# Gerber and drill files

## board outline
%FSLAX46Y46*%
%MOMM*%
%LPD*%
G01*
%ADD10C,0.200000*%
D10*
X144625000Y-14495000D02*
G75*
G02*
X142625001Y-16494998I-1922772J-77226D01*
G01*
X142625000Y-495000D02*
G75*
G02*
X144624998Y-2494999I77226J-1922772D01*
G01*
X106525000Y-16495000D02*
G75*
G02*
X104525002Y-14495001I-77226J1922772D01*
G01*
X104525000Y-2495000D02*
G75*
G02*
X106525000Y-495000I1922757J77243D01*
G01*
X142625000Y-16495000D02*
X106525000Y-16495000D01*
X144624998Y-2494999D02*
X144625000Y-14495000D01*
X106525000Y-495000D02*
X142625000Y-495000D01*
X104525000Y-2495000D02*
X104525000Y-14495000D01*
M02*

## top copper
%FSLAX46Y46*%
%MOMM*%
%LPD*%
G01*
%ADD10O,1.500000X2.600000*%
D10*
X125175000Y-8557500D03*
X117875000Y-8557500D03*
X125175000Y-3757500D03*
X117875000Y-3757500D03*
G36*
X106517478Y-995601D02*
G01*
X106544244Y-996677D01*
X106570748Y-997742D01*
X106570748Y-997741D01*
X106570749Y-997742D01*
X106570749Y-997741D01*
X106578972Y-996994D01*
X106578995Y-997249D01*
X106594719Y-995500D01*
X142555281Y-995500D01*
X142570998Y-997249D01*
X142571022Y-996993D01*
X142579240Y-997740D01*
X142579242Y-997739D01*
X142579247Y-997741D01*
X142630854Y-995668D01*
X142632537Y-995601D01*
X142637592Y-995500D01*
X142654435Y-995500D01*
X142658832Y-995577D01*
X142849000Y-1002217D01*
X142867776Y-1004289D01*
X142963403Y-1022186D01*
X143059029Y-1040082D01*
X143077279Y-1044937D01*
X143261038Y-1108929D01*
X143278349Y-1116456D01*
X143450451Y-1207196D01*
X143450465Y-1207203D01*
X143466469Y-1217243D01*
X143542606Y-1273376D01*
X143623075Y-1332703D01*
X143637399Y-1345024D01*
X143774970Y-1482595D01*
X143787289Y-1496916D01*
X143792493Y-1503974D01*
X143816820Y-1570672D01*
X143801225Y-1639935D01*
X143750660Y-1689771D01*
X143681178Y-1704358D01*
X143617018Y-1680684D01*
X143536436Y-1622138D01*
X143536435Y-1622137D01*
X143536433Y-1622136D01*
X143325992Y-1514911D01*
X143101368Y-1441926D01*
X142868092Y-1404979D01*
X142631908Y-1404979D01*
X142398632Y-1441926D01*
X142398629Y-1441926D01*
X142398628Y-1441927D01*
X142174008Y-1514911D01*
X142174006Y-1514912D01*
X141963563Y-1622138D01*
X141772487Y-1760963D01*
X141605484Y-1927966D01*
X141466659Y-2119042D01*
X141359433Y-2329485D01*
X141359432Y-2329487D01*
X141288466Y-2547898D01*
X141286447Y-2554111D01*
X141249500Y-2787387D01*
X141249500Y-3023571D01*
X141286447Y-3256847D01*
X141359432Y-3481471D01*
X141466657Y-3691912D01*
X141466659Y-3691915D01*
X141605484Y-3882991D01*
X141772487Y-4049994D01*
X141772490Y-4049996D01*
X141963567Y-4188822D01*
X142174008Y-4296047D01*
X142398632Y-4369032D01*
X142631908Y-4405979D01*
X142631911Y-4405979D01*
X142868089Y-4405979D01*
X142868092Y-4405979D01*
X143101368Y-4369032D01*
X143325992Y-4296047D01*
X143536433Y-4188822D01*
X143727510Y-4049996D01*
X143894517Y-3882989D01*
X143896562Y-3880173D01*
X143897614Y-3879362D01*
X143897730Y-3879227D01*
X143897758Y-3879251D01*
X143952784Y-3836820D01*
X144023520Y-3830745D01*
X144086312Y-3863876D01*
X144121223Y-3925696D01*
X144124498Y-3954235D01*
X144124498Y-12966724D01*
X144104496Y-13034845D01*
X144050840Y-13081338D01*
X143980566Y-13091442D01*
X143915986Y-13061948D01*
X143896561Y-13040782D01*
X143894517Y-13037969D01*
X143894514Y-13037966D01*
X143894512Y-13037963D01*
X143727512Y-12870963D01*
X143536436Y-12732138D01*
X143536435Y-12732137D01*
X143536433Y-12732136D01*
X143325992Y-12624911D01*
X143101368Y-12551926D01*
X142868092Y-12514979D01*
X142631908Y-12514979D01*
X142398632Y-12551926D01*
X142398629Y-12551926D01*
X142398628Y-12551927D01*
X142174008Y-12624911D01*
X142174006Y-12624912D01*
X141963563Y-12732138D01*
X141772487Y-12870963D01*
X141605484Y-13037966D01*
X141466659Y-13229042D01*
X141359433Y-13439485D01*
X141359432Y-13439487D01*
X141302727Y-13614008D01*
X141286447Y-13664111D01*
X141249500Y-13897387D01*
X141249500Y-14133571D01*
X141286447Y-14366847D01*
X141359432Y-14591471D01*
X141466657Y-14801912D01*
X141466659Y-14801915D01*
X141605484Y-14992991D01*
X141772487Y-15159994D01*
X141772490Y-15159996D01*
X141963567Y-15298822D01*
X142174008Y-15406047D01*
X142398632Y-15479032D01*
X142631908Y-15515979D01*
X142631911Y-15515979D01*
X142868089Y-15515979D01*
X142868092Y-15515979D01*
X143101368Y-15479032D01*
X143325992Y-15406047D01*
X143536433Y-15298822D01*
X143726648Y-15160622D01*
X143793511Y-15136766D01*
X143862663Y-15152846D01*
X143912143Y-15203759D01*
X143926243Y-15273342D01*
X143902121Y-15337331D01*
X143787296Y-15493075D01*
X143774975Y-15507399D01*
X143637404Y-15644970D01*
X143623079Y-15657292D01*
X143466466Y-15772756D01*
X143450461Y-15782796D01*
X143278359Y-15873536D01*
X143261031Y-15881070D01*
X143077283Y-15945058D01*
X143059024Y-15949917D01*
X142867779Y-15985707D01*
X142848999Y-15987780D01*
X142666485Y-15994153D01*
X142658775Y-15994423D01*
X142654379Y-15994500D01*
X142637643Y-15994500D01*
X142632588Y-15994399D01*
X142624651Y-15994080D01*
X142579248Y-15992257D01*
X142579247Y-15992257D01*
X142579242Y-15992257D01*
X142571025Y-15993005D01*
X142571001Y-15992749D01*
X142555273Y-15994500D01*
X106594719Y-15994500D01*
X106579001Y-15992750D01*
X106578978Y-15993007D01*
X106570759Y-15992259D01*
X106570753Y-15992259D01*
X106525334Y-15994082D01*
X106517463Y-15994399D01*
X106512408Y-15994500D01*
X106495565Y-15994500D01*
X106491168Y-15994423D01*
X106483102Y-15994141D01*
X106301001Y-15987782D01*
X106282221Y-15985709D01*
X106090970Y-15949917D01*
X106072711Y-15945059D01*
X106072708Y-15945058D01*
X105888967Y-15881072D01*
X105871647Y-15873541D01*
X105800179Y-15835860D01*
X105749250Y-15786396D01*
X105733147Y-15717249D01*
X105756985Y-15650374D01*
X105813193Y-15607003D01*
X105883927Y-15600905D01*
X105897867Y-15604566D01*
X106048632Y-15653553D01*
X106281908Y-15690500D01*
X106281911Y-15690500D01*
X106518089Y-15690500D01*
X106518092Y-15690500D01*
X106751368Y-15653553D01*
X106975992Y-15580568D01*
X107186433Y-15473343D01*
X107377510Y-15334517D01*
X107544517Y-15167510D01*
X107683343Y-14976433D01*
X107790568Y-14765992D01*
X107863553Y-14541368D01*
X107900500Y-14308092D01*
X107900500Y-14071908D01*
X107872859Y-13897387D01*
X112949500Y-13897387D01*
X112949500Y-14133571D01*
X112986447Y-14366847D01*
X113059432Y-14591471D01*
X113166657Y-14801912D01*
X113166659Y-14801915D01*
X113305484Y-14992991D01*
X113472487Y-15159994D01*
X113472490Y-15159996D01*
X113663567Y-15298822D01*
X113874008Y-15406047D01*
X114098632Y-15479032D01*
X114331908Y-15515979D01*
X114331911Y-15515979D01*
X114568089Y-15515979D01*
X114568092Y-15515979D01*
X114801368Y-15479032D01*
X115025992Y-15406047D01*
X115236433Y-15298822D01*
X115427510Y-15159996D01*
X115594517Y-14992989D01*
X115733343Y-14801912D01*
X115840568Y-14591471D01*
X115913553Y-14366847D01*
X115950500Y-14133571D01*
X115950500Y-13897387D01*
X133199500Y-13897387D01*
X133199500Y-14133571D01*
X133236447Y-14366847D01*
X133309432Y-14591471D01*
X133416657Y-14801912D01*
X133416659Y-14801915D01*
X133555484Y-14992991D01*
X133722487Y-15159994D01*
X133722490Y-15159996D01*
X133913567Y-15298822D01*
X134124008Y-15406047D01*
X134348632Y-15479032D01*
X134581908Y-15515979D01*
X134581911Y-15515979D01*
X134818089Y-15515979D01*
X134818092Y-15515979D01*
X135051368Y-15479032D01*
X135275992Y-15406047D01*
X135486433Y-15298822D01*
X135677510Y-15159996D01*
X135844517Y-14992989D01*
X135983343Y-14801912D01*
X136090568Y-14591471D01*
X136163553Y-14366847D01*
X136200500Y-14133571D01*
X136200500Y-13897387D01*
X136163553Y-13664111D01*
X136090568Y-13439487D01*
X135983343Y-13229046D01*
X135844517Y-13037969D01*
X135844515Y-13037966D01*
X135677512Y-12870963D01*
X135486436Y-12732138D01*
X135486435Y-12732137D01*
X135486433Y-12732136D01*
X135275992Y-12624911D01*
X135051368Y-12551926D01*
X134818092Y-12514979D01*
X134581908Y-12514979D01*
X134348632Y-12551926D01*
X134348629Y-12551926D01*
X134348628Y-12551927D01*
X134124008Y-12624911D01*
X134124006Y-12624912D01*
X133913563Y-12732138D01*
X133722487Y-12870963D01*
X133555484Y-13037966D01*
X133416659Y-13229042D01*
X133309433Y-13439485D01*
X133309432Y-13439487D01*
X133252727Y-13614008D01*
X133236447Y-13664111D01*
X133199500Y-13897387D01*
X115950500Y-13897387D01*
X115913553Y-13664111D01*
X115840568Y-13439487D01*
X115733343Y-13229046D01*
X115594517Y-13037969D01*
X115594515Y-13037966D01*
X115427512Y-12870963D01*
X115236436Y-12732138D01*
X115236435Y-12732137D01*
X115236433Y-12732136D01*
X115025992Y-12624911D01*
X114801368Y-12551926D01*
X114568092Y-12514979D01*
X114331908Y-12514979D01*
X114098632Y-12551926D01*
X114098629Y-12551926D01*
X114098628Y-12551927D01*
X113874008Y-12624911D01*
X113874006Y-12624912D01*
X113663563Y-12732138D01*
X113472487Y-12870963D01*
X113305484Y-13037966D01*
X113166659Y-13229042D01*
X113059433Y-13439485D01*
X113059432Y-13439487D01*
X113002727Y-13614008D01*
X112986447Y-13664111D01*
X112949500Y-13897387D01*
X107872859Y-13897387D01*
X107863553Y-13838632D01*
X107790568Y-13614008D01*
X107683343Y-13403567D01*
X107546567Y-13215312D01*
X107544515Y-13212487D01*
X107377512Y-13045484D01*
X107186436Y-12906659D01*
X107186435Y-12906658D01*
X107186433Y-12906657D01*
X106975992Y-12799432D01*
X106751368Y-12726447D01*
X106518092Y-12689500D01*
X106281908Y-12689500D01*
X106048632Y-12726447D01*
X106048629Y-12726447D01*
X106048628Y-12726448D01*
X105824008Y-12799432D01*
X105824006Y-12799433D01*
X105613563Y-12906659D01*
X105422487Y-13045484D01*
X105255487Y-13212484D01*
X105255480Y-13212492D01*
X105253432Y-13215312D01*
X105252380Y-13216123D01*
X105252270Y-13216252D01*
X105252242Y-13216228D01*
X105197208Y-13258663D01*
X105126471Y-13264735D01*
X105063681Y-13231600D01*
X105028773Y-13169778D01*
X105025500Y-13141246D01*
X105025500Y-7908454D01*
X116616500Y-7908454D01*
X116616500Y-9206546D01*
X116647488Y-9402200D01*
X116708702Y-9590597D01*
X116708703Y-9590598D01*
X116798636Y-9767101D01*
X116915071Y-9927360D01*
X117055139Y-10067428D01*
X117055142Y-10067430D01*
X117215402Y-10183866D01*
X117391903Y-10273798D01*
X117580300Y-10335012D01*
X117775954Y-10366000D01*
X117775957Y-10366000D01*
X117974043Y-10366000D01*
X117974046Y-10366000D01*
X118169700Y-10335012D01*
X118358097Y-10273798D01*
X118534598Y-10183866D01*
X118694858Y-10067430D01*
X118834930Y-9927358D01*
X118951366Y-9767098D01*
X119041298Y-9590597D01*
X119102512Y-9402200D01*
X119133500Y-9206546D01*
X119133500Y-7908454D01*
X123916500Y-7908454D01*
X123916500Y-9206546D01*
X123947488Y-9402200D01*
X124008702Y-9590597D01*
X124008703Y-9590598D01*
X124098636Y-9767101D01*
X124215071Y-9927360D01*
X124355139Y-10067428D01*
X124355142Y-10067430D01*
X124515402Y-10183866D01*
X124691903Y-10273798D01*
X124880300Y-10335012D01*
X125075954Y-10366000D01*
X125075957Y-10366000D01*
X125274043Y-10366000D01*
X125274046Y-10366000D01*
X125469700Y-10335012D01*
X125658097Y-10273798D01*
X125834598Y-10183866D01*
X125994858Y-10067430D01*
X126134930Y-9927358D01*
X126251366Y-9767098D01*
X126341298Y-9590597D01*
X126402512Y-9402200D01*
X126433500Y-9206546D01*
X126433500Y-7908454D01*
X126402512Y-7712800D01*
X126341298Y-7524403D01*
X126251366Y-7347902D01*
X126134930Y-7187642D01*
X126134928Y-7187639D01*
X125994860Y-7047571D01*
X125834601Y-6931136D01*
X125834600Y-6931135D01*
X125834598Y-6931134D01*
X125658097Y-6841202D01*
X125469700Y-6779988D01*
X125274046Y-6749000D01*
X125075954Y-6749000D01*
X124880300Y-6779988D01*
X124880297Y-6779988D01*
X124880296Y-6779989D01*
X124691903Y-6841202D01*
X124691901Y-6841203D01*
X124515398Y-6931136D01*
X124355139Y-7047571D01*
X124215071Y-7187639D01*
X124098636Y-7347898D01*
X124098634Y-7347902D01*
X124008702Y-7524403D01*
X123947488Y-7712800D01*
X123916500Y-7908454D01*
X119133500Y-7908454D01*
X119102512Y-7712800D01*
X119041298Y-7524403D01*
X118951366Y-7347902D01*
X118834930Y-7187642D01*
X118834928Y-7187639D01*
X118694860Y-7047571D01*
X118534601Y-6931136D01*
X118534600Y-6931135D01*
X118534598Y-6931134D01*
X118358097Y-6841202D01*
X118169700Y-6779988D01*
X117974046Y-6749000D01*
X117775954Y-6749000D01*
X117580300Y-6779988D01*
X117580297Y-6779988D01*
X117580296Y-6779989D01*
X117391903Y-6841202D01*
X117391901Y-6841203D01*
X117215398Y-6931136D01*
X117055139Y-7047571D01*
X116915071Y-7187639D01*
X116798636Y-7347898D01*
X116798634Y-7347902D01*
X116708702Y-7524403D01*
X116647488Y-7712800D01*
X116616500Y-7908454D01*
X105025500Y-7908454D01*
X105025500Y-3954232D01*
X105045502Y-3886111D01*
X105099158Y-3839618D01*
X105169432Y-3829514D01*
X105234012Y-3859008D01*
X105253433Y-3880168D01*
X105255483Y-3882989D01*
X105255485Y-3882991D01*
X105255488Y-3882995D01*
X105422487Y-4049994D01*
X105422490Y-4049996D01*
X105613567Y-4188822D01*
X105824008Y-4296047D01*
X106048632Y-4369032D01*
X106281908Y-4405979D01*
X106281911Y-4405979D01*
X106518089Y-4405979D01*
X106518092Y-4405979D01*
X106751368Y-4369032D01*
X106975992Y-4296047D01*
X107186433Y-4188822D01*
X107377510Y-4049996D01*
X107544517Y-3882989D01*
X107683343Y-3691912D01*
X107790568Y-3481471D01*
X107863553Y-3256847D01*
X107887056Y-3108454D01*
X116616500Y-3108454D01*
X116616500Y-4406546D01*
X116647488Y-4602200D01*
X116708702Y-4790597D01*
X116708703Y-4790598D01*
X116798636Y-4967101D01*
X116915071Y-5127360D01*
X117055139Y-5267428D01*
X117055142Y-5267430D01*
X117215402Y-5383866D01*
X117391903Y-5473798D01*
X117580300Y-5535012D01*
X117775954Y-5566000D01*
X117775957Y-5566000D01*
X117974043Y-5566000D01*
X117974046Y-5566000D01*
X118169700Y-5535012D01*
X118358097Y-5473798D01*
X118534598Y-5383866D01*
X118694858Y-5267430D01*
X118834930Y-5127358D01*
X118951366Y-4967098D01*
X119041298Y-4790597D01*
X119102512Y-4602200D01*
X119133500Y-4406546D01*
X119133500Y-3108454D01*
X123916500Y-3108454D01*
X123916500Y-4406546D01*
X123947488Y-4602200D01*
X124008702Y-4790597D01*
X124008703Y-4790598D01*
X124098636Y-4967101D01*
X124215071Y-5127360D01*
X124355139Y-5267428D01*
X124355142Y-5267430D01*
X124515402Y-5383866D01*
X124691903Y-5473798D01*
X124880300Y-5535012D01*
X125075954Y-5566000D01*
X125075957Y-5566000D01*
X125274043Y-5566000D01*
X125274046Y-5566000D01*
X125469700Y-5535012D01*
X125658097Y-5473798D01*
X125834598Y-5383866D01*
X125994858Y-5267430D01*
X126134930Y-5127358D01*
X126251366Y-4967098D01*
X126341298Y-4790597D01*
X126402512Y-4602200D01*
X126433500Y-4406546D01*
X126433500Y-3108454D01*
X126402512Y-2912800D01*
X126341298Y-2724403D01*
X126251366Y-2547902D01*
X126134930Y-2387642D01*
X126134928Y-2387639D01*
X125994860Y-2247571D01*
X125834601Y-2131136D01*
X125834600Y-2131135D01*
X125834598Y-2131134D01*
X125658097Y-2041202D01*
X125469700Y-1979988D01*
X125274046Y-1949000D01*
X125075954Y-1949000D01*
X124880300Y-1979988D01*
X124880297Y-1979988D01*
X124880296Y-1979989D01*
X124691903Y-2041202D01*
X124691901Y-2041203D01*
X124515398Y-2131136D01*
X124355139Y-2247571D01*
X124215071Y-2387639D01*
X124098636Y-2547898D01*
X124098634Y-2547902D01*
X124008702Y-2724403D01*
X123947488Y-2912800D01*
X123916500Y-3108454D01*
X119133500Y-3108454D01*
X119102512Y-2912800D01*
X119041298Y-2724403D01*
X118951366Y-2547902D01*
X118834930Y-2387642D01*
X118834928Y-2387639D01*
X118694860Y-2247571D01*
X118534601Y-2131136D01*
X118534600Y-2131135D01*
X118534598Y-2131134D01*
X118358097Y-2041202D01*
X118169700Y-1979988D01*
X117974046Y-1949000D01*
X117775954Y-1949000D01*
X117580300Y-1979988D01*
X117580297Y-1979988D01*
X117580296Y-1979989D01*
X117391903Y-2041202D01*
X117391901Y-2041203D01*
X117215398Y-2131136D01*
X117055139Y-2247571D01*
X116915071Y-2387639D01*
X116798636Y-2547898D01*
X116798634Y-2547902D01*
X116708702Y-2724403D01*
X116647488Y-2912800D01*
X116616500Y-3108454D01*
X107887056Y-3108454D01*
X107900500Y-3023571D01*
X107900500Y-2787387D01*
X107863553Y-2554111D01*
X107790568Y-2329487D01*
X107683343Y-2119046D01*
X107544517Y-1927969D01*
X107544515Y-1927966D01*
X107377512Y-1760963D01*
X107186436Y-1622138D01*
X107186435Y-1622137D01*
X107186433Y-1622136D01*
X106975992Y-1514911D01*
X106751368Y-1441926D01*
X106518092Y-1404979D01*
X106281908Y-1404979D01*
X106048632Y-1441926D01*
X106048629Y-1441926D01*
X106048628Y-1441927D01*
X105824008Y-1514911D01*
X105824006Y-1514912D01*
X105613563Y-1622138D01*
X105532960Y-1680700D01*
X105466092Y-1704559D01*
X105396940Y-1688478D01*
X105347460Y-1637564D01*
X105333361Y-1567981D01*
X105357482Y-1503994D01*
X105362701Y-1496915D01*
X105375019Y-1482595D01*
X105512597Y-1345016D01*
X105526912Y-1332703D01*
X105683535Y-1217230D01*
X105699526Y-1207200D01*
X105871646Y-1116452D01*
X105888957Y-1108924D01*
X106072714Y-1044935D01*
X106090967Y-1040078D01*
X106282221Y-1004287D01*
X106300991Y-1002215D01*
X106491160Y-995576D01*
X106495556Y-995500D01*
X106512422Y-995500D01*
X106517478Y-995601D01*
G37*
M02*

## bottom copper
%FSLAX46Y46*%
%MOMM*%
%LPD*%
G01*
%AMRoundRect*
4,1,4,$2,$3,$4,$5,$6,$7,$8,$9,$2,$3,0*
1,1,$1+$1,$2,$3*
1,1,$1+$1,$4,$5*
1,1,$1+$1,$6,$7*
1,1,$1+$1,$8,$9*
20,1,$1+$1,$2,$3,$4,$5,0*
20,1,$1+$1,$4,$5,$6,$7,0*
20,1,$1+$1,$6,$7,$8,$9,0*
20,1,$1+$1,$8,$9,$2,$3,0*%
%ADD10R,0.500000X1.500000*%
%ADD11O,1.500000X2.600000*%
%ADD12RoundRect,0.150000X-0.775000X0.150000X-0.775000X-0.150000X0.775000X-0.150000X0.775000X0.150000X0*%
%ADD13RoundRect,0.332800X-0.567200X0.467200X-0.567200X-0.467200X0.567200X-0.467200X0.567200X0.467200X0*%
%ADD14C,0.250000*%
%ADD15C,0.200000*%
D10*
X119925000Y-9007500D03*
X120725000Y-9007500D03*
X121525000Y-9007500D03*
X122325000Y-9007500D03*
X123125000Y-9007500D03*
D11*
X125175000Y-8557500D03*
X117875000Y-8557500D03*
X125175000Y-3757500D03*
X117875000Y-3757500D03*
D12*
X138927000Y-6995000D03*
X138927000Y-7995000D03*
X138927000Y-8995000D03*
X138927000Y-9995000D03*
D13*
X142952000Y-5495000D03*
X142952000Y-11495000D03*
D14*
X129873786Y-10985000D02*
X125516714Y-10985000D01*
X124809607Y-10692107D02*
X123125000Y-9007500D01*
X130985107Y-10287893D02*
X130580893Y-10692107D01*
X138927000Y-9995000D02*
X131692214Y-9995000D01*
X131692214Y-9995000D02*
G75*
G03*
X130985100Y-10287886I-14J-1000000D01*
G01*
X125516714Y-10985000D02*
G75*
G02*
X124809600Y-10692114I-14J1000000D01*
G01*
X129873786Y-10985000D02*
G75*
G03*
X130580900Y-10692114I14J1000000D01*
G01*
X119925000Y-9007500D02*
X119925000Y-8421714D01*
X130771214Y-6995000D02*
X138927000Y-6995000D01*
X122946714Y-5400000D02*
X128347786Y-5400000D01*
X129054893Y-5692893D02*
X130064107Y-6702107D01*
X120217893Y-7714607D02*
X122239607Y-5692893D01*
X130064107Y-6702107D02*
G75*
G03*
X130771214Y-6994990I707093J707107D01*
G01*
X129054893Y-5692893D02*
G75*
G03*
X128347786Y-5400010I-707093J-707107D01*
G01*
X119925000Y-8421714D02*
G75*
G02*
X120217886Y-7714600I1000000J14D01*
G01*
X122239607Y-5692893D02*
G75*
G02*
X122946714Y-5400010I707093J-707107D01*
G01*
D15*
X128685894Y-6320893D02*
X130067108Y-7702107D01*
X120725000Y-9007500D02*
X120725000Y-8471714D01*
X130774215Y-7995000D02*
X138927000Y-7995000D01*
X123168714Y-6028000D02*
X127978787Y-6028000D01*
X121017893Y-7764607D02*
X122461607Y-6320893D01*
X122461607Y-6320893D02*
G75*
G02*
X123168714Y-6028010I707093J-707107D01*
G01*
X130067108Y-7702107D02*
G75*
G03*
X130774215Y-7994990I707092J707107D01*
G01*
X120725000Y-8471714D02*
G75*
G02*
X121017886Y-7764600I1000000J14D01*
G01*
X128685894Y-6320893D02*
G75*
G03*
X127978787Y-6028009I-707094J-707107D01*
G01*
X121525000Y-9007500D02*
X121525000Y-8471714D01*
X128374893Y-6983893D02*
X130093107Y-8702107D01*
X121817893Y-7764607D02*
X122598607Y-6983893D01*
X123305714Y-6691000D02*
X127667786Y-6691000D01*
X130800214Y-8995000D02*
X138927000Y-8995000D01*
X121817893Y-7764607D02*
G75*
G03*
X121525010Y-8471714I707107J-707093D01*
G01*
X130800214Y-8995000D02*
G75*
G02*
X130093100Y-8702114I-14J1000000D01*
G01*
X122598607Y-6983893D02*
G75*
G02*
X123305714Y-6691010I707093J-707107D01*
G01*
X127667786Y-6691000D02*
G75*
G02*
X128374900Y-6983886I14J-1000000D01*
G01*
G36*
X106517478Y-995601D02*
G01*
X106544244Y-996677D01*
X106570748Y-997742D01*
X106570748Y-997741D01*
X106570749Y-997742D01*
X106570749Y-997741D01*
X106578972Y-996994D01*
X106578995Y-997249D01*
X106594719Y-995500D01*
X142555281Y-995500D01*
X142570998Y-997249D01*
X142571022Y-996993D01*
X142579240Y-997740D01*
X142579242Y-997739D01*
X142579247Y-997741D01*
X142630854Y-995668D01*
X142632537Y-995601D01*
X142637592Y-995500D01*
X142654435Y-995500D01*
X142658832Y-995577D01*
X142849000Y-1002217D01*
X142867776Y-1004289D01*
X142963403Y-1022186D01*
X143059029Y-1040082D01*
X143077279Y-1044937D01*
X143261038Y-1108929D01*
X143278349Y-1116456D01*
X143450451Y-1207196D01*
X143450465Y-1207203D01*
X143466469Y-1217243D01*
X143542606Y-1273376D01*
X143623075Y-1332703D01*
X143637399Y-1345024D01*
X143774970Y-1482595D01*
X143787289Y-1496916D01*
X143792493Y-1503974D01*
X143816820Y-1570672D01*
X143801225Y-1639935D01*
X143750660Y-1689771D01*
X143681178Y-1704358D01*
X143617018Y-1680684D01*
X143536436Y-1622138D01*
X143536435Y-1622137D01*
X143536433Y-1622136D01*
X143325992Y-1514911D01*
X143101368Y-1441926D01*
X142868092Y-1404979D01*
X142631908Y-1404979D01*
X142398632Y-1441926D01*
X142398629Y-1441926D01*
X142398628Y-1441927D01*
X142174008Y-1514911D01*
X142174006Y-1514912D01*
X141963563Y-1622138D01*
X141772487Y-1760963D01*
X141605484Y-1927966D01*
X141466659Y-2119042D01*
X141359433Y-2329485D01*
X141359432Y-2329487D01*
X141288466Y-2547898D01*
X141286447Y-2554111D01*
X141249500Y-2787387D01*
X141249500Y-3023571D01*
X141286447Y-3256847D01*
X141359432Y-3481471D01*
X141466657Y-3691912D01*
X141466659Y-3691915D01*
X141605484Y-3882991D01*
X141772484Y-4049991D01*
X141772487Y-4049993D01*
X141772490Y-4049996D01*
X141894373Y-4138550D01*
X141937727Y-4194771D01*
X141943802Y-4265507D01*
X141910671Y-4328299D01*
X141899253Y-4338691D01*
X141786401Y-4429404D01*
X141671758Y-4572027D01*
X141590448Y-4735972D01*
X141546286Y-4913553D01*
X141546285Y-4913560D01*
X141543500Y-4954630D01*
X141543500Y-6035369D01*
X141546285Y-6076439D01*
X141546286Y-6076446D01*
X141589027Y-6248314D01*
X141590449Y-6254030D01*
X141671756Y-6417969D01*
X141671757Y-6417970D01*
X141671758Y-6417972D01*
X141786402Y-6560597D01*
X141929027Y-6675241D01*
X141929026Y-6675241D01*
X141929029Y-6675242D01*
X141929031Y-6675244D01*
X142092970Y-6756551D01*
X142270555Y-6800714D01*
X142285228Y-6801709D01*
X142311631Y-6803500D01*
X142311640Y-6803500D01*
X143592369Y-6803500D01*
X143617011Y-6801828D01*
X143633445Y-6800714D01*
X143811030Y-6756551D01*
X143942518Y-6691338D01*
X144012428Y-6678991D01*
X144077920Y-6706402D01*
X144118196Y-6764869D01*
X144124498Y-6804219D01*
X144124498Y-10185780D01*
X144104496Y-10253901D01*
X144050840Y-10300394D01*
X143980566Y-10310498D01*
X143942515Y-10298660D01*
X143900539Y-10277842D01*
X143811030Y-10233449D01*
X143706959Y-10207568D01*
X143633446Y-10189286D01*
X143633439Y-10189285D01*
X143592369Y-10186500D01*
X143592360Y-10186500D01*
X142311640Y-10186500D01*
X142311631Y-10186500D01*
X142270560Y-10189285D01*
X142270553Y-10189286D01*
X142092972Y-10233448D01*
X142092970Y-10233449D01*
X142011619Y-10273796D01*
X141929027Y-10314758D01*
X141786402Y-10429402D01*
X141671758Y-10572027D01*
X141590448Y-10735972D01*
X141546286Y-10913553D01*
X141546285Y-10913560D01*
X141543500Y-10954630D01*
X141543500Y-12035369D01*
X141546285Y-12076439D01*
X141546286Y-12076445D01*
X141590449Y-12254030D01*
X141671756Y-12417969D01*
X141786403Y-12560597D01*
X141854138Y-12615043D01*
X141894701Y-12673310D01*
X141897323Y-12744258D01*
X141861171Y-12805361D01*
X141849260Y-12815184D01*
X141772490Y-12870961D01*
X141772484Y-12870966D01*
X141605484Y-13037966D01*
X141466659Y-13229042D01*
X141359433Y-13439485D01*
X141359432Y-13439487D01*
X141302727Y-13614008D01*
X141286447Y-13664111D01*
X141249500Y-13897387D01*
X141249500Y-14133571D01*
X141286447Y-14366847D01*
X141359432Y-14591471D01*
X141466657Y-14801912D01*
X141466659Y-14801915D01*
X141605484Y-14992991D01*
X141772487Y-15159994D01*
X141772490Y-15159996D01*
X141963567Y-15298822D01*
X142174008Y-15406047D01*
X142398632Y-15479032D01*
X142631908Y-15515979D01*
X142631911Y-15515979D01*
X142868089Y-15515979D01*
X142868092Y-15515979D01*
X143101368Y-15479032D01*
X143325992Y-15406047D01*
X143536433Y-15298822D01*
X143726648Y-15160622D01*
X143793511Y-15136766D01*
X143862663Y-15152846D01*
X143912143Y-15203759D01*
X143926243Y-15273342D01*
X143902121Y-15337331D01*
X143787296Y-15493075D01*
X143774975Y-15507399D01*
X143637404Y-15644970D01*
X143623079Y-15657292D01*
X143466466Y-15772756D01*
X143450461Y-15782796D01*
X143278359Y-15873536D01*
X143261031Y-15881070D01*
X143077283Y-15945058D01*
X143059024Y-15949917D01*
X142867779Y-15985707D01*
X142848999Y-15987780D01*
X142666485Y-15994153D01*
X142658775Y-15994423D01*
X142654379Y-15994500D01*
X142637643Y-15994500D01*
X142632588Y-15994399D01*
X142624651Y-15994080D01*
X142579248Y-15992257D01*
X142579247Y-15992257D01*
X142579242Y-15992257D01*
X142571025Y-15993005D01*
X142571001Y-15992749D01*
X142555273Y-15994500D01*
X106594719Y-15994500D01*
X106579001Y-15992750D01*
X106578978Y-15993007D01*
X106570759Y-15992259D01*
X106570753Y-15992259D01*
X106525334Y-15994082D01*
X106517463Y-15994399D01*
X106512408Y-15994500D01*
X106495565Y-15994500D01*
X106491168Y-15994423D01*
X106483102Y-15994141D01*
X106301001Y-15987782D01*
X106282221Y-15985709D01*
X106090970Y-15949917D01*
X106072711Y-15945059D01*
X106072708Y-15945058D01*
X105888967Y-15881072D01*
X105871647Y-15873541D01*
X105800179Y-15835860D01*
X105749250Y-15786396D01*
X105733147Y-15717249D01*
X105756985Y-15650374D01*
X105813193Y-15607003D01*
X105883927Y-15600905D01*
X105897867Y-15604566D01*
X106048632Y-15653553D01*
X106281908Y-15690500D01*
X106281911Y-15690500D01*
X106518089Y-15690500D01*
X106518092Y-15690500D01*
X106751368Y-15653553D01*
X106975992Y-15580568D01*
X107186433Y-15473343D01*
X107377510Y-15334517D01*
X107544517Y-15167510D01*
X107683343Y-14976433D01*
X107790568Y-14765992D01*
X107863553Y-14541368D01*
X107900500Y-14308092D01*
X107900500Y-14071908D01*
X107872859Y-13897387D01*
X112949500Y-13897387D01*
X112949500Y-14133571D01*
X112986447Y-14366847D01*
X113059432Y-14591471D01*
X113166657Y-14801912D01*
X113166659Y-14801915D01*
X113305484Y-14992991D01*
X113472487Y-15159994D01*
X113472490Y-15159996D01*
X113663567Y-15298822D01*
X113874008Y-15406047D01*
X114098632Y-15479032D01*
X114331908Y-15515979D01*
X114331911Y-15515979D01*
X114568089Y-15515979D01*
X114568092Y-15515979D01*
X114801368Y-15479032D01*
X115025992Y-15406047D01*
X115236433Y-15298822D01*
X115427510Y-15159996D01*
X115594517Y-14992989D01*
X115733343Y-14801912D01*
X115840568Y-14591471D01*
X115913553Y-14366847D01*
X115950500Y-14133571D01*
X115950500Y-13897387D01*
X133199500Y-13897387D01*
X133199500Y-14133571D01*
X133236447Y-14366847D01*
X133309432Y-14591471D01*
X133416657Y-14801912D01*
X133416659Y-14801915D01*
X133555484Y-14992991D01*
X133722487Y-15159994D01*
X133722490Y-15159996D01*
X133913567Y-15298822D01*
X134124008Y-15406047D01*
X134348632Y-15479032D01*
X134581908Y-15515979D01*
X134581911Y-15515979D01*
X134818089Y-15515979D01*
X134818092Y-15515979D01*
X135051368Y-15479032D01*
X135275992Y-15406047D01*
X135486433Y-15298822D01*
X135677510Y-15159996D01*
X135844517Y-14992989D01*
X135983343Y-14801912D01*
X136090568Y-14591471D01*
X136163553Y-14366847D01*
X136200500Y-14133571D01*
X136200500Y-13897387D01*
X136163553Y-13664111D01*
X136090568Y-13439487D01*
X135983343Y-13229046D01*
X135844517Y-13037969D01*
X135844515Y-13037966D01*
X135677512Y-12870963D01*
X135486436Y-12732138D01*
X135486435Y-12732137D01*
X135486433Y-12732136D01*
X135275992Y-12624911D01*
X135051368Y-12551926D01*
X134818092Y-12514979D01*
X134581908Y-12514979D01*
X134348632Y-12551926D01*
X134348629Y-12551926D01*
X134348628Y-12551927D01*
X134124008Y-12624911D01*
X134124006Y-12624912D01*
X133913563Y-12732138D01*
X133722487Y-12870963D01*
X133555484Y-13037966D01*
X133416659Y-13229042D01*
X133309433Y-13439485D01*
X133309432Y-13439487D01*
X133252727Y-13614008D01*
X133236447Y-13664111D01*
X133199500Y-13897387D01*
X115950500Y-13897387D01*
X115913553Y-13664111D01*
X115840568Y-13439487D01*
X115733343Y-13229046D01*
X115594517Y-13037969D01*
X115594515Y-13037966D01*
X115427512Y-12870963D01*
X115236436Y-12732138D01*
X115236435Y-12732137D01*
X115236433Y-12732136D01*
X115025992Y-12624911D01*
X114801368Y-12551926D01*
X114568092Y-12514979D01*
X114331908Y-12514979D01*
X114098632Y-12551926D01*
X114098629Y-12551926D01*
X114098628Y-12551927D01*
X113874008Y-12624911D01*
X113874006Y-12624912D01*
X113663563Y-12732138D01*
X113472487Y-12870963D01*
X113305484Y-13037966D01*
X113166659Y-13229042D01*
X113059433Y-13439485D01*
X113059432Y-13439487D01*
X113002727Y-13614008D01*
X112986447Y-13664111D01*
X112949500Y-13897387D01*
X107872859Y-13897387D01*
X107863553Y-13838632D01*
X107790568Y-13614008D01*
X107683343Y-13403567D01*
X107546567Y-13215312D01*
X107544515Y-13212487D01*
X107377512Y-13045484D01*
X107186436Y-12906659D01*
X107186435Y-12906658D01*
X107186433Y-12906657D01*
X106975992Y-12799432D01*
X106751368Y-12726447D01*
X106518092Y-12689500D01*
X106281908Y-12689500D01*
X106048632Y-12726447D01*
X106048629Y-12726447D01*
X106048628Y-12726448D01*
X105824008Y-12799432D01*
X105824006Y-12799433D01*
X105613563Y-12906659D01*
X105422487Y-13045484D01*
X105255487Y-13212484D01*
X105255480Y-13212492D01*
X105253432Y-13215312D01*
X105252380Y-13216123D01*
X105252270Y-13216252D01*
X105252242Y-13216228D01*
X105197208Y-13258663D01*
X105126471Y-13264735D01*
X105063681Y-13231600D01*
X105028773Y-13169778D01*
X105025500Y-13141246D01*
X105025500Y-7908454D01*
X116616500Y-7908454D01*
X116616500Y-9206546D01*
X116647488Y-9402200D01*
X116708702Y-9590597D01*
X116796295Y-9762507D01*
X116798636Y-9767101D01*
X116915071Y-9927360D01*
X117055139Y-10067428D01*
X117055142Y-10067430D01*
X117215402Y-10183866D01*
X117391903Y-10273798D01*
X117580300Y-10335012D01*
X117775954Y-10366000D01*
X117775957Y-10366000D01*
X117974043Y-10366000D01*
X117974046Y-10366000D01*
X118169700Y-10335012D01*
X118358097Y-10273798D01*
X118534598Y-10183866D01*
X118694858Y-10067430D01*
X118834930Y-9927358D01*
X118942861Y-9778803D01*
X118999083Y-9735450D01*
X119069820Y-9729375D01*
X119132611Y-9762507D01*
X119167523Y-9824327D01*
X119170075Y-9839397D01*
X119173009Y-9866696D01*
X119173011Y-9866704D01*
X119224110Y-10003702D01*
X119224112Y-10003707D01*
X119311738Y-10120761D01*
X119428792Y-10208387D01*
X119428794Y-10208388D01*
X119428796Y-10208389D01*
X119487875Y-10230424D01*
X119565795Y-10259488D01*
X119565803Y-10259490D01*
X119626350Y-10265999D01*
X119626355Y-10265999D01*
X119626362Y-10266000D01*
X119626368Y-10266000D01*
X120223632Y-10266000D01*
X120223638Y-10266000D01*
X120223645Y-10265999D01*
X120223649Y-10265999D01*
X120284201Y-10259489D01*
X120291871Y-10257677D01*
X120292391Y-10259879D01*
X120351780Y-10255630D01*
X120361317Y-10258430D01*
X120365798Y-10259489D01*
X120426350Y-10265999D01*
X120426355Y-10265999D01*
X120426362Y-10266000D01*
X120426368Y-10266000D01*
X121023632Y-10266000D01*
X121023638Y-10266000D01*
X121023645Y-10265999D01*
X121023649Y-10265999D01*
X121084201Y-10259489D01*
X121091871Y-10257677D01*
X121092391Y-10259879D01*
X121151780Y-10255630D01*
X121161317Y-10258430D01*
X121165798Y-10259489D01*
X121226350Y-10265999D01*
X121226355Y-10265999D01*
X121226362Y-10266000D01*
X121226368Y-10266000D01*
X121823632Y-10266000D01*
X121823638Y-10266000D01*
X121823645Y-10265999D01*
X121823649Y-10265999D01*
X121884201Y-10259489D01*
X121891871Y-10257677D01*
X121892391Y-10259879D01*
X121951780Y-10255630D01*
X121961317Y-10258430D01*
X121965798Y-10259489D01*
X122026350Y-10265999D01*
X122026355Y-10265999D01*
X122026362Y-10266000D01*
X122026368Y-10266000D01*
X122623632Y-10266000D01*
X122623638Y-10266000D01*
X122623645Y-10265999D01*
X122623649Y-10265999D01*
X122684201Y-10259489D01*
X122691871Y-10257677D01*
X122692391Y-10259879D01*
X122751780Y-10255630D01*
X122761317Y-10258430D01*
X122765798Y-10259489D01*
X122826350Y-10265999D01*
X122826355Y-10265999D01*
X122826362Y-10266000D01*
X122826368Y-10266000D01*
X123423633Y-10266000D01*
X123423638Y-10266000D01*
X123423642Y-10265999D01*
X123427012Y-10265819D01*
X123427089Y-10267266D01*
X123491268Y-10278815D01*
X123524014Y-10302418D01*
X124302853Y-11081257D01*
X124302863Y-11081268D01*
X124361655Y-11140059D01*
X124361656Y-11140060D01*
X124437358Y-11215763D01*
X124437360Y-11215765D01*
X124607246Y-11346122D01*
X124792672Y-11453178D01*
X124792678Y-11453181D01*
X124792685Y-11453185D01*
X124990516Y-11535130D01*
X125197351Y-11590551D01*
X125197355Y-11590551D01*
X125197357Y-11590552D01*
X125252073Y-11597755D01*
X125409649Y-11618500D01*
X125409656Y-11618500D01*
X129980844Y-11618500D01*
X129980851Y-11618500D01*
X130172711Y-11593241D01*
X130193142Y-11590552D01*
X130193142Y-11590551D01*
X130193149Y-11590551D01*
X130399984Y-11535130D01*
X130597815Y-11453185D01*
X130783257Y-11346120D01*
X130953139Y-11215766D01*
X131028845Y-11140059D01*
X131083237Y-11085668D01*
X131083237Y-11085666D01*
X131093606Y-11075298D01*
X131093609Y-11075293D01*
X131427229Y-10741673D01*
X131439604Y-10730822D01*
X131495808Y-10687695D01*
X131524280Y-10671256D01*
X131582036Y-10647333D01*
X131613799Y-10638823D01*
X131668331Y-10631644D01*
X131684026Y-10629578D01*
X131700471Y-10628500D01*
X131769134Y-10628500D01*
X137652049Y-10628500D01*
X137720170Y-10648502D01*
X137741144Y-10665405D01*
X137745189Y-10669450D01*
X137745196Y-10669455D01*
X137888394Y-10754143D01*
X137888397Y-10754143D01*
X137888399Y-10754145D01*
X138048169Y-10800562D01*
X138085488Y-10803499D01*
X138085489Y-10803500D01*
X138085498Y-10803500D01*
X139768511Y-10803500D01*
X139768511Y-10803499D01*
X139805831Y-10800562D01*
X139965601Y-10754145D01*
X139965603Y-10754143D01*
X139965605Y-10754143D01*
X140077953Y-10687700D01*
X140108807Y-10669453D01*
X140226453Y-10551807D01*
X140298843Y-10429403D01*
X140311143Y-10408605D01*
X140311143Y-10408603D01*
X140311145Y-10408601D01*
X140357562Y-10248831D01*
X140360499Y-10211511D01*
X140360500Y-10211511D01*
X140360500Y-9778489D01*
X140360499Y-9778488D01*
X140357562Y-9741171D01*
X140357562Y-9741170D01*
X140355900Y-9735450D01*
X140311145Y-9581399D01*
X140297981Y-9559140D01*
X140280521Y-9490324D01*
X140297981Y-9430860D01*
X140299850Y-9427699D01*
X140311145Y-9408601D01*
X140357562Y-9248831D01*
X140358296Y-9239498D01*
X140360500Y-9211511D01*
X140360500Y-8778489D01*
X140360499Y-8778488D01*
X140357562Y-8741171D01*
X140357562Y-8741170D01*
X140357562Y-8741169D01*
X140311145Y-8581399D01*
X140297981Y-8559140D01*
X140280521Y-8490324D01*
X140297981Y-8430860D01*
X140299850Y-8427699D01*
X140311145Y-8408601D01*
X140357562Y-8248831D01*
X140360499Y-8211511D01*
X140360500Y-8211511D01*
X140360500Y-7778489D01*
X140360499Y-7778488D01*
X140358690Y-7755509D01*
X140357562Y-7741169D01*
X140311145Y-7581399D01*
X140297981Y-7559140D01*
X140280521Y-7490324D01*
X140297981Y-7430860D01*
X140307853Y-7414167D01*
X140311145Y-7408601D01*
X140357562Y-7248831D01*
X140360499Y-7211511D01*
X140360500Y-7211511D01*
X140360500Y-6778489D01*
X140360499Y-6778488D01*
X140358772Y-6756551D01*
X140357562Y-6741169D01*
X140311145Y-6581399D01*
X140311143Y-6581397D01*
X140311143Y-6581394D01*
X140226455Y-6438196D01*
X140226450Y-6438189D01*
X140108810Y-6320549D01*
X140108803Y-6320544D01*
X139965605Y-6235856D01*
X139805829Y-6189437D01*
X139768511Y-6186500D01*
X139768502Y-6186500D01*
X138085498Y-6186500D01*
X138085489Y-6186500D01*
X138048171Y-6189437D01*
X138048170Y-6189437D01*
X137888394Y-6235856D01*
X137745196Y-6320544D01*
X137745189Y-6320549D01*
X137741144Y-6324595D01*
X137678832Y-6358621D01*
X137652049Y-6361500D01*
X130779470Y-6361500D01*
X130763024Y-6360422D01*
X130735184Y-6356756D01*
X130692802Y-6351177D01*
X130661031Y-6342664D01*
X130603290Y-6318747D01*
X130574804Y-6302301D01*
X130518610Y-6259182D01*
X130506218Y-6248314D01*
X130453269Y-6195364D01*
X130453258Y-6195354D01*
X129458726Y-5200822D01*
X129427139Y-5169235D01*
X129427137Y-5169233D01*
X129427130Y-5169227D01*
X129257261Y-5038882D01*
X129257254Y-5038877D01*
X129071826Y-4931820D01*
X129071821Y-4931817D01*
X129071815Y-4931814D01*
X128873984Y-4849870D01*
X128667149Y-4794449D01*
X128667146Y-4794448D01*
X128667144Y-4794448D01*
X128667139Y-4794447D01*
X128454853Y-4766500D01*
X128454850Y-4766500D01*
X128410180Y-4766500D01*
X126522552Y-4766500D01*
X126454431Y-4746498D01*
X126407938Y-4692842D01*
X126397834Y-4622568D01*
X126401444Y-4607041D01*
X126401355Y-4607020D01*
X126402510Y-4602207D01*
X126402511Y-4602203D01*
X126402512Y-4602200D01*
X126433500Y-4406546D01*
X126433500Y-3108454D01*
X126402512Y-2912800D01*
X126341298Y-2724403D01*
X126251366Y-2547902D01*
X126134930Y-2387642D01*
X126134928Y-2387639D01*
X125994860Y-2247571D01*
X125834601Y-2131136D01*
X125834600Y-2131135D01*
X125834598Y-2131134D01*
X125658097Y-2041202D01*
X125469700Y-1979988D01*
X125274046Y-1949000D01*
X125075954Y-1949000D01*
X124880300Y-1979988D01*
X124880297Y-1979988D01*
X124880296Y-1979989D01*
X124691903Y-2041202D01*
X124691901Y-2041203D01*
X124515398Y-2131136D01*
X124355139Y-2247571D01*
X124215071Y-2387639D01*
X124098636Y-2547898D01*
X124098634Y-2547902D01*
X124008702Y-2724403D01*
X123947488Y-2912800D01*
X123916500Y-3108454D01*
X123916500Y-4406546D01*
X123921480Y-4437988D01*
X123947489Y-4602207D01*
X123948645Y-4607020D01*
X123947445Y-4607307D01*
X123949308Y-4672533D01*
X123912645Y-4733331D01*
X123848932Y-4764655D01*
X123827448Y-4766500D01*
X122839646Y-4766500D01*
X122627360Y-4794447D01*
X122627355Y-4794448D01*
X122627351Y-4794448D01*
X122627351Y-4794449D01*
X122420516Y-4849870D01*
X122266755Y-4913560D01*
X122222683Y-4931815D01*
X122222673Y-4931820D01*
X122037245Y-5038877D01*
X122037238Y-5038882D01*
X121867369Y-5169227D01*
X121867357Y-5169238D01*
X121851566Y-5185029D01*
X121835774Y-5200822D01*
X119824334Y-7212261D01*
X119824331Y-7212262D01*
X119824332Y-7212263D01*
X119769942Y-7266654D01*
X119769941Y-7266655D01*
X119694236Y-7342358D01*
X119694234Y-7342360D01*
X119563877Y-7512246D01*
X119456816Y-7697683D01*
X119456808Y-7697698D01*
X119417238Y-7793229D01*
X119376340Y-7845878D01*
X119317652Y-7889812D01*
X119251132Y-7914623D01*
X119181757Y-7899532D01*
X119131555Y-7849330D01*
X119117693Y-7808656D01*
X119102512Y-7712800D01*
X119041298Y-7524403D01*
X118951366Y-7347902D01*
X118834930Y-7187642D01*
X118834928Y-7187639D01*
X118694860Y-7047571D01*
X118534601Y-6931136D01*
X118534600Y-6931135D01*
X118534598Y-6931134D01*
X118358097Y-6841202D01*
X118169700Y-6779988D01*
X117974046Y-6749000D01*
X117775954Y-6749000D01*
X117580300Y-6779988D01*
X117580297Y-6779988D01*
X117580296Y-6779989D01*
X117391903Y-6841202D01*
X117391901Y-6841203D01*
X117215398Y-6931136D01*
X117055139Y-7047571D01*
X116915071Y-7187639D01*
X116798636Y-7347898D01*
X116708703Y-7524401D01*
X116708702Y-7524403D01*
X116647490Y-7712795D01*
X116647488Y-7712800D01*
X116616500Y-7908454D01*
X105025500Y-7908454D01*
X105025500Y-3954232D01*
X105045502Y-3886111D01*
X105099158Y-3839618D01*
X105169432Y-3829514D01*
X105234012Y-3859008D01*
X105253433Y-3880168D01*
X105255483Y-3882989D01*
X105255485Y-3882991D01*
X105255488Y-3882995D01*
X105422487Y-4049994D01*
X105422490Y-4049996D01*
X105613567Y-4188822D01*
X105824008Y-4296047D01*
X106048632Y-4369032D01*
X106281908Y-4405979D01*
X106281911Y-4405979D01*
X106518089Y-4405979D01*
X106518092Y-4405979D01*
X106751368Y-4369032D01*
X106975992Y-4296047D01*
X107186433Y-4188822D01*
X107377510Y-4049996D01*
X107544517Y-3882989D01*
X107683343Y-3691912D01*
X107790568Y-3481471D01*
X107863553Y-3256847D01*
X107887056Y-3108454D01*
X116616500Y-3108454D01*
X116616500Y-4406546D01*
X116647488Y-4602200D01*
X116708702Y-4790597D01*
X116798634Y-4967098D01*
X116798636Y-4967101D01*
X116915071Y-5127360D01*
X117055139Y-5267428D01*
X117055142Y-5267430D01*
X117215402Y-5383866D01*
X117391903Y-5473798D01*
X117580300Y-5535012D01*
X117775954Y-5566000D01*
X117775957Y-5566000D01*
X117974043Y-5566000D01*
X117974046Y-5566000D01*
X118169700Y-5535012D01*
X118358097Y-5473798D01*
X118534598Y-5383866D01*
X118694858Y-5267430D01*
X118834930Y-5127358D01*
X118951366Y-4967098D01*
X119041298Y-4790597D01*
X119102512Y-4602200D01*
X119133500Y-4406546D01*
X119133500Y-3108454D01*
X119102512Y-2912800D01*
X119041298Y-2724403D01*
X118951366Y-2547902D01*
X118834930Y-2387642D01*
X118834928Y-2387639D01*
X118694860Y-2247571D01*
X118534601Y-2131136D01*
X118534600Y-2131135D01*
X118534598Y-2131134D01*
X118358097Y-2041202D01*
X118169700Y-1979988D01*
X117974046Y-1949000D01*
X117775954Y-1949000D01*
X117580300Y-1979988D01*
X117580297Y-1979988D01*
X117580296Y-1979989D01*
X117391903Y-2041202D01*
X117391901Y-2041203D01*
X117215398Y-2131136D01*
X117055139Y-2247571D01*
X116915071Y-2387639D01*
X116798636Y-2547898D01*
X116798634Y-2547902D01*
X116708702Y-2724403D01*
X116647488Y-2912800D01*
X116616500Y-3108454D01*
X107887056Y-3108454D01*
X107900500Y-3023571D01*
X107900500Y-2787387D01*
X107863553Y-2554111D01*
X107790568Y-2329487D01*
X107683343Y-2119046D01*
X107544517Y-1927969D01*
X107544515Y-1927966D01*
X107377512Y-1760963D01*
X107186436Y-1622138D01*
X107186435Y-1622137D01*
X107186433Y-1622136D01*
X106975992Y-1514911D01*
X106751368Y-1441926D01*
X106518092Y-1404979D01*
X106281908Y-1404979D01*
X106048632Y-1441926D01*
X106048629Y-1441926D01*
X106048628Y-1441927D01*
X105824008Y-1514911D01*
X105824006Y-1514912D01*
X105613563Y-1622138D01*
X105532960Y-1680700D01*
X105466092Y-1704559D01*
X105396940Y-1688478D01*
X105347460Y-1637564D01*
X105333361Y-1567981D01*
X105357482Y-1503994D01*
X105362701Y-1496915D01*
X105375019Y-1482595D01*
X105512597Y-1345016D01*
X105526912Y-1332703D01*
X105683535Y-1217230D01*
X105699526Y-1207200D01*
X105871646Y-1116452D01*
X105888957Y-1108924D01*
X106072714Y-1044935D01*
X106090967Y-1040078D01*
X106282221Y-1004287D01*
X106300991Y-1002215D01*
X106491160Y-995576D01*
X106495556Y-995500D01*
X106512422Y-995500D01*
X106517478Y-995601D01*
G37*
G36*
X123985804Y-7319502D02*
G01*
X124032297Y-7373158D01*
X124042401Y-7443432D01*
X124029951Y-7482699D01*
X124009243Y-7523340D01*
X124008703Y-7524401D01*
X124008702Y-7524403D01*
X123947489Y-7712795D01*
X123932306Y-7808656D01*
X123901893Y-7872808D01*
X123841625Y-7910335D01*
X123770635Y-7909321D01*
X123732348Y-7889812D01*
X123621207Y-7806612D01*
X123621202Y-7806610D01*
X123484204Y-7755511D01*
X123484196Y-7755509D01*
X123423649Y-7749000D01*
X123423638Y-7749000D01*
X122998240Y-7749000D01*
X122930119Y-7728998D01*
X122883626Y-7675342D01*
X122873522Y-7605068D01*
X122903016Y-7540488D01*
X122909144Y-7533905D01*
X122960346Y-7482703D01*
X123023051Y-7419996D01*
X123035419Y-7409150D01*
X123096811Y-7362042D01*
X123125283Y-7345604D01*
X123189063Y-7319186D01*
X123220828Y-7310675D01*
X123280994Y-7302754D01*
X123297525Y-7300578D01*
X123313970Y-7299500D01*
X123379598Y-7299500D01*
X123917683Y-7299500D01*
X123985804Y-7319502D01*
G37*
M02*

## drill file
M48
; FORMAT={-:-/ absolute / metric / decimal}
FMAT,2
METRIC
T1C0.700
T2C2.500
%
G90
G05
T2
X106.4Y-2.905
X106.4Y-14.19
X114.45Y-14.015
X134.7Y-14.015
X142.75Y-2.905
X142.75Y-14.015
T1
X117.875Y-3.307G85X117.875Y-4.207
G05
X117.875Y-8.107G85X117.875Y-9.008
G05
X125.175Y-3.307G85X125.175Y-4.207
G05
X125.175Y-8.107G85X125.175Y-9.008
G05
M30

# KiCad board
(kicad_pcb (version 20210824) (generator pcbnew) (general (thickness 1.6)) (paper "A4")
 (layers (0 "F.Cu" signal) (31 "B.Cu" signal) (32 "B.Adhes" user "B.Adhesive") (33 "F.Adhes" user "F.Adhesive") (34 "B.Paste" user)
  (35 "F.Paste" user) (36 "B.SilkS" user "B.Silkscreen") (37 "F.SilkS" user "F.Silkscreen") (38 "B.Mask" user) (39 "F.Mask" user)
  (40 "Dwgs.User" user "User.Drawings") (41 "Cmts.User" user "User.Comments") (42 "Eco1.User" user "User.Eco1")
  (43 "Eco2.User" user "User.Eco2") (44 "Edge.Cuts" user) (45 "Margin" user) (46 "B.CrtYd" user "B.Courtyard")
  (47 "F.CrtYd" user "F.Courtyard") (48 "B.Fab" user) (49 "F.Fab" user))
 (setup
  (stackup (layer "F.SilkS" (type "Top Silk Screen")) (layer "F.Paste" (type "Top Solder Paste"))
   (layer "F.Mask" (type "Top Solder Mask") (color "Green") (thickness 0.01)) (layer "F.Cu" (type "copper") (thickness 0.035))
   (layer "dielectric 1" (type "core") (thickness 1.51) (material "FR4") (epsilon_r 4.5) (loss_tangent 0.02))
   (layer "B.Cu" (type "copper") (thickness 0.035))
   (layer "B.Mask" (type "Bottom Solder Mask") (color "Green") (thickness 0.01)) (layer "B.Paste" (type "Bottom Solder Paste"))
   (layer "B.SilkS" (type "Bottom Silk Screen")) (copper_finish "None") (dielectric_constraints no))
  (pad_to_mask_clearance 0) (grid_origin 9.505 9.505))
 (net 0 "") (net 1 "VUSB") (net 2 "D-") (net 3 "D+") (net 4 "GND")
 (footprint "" (layer "F.Cu") (at 136.255 14.205)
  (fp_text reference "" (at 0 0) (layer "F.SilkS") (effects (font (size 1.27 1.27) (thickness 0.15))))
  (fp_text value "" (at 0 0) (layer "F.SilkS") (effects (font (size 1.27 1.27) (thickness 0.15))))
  (pad "" np_thru_hole circle (at -1.555 -0.189521) (size 2.5 2.5) (drill 2.5) (layers F&B.Cu *.Mask)))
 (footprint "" (layer "F.Cu") (at 94.555 1.535)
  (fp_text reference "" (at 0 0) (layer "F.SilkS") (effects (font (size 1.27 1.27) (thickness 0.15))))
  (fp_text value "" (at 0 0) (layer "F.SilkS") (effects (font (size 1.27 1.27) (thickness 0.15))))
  (pad "" np_thru_hole circle (at 11.845 1.370479) (size 2.5 2.5) (drill 2.5) (layers F&B.Cu *.Mask)))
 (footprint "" (layer "F.Cu") (at 147.015 3.065)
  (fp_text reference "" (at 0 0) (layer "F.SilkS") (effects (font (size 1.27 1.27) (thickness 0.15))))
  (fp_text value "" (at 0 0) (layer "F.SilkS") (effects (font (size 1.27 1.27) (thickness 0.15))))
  (pad "" np_thru_hole circle (at -4.265 -0.159521) (size 2.5 2.5) (drill 2.5) (layers F&B.Cu *.Mask)))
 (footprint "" (layer "F.Cu") (at 94.295 7.445633)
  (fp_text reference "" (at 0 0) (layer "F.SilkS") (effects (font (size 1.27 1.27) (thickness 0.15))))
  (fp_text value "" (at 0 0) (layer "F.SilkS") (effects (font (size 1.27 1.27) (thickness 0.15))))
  (pad "" np_thru_hole circle (at 12.105 6.744367) (size 2.5 2.5) (drill 2.5) (layers F&B.Cu *.Mask)))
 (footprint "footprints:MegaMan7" (layer "F.Cu") (at 109.650838 8.415023)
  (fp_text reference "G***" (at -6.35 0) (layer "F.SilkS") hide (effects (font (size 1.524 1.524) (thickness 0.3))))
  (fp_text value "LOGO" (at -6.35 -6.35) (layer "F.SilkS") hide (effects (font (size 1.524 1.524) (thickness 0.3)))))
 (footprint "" (layer "F.Cu") (at 112.225 13.965)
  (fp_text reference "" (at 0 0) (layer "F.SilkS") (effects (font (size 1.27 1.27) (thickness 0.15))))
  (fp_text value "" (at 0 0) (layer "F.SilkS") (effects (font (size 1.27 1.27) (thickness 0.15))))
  (pad "" np_thru_hole circle (at 2.225 0.050479) (size 2.5 2.5) (drill 2.5) (layers F&B.Cu *.Mask)))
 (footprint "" (layer "F.Cu") (at 130.75 14.19)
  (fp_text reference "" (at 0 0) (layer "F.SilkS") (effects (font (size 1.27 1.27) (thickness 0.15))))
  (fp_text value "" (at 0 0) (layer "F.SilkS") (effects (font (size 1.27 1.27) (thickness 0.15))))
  (pad "" np_thru_hole circle (at 12 -0.174521) (size 2.5 2.5) (drill 2.5) (layers F&B.Cu *.Mask)))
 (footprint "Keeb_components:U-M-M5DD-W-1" (layer "B.Cu") (at 121.525 3.7575 180)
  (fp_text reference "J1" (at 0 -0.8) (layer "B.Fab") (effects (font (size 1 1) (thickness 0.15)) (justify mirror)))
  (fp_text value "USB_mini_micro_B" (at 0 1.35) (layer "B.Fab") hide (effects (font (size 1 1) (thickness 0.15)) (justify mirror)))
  (pad "1" smd rect locked (at 1.6 -5.25) (size 0.5 1.5) (layers "B.Cu" "B.Paste" "B.Mask") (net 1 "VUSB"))
  (pad "2" smd rect locked (at 0.8 -5.25) (size 0.5 1.5) (layers "B.Cu" "B.Paste" "B.Mask") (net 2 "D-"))
  (pad "3" smd rect locked (at 0 -5.25) (size 0.5 1.5) (layers "B.Cu" "B.Paste" "B.Mask") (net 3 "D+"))
  (pad "4" smd rect locked (at -0.8 -5.25) (size 0.5 1.5) (layers "B.Cu" "B.Paste" "B.Mask"))
  (pad "5" smd rect locked (at -1.6 -5.25) (size 0.5 1.5) (layers "B.Cu" "B.Paste" "B.Mask") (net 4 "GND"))
  (pad "6" thru_hole oval locked (at -3.65 -4.8) (size 1.5 2.6) (drill oval 0.7 1.6) (layers *.Cu *.Mask))
  (pad "6" thru_hole oval locked (at 3.65 -4.8) (size 1.5 2.6) (drill oval 0.7 1.6) (layers *.Cu *.Mask))
  (pad "6" thru_hole oval locked (at -3.65 0) (size 1.5 2.6) (drill oval 0.7 1.6) (layers *.Cu *.Mask))
  (pad "6" thru_hole oval locked (at 3.65 0) (size 1.5 2.6) (drill oval 0.7 1.6) (layers *.Cu *.Mask)))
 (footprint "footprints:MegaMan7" (layer "B.Cu") (at 109.67284 8.39588 180)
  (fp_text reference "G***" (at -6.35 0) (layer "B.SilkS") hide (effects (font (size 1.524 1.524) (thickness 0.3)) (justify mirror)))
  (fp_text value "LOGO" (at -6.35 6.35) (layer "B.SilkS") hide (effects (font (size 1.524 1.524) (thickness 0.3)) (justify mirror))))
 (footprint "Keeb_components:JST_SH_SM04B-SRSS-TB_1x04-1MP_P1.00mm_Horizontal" (layer "B.Cu") (at 141.077 8.495 -90)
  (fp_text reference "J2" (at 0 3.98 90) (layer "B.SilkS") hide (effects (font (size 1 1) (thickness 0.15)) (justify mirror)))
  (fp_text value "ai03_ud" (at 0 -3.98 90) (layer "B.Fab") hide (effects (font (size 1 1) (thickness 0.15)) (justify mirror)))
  (pad "1" smd roundrect locked (at -1.5 2.15 270) (size 0.6 1.85) (layers "B.Cu" "B.Paste" "B.Mask") (roundrect_rratio 0.25) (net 1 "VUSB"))
  (pad "2" smd roundrect locked (at -0.5 2.15 270) (size 0.6 1.85) (layers "B.Cu" "B.Paste" "B.Mask") (roundrect_rratio 0.25) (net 2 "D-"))
  (pad "3" smd roundrect locked (at 0.5 2.15 270) (size 0.6 1.85) (layers "B.Cu" "B.Paste" "B.Mask") (roundrect_rratio 0.25) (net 3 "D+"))
  (pad "4" smd roundrect locked (at 1.5 2.15 270) (size 0.6 1.85) (layers "B.Cu" "B.Paste" "B.Mask") (roundrect_rratio 0.25) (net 4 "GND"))
  (pad "MP" smd roundrect locked (at -3 -1.875 270) (size 1.6 1.8) (layers "B.Cu" "B.Paste" "B.Mask") (roundrect_rratio 0.208))
  (pad "MP" smd roundrect locked (at 3 -1.875 270) (size 1.6 1.8) (layers "B.Cu" "B.Paste" "B.Mask") (roundrect_rratio 0.208)))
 (gr_arc (start 142.702228 14.572226) (end 144.625 14.495) (angle 94.6) (layer "Edge.Cuts") (width 0.2))
 (gr_arc (start 142.702226 2.417772) (end 142.625 0.495) (angle 94.6) (layer "Edge.Cuts") (width 0.2))
 (gr_arc (start 106.447774 14.572228) (end 106.525 16.495) (angle 94.6) (layer "Edge.Cuts") (width 0.2))
 (gr_arc (start 106.447757 2.417757) (end 104.525 2.495) (angle 94.60101756) (layer "Edge.Cuts") (width 0.2))
 (gr_line (start 142.625 16.495) (end 106.525 16.495) (layer "Edge.Cuts") (width 0.2))
 (gr_line (start 144.624998 2.494999) (end 144.625 14.495) (layer "Edge.Cuts") (width 0.2))
 (gr_line (start 106.525 0.495) (end 142.625 0.495) (layer "Edge.Cuts") (width 0.2))
 (gr_line (start 104.525 2.495) (end 104.525 14.495) (layer "Edge.Cuts") (width 0.2))
 (segment (start 129.873786 10.985) (end 125.516714 10.985) (width 0.25) (layer "B.Cu") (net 4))
 (segment (start 124.809607 10.692107) (end 123.125 9.0075) (width 0.25) (layer "B.Cu") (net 4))
 (segment (start 130.985107 10.287893) (end 130.580893 10.692107) (width 0.25) (layer "B.Cu") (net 4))
 (segment (start 138.927 9.995) (end 131.692214 9.995) (width 0.25) (layer "B.Cu") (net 4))
 (arc (start 131.692214 9.995) (mid 131.309531 10.07112) (end 130.985107 10.287893) (width 0.25) (layer "B.Cu") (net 4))
 (arc (start 125.516714 10.985) (mid 125.134031 10.90888) (end 124.809607 10.692107) (width 0.25) (layer "B.Cu") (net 4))
 (arc (start 129.873786 10.985) (mid 130.256469 10.90888) (end 130.580893 10.692107) (width 0.25) (layer "B.Cu") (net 4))
 (segment (start 119.925 9.0075) (end 119.925 8.421714) (width 0.25) (layer "B.Cu") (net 1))
 (segment (start 130.771214 6.995) (end 138.927 6.995) (width 0.25) (layer "B.Cu") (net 1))
 (segment (start 122.946714 5.4) (end 128.347786 5.4) (width 0.25) (layer "B.Cu") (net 1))
 (segment (start 129.054893 5.692893) (end 130.064107 6.702107) (width 0.25) (layer "B.Cu") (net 1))
 (segment (start 120.217893 7.714607) (end 122.239607 5.692893) (width 0.25) (layer "B.Cu") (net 1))
 (arc (start 130.064107 6.702107) (mid 130.38853 6.91888) (end 130.771214 6.995) (width 0.25) (layer "B.Cu") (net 1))
 (arc (start 129.054893 5.692893) (mid 128.73047 5.47612) (end 128.347786 5.4) (width 0.25) (layer "B.Cu") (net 1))
 (arc (start 119.925 8.421714) (mid 120.00112 8.039031) (end 120.217893 7.714607) (width 0.25) (layer "B.Cu") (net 1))
 (arc (start 122.239607 5.692893) (mid 122.56403 5.47612) (end 122.946714 5.4) (width 0.25) (layer "B.Cu") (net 1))
 (segment (start 128.685894 6.320893) (end 130.067108 7.702107) (width 0.2) (layer "B.Cu") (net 2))
 (segment (start 120.725 9.0075) (end 120.725 8.471714) (width 0.2) (layer "B.Cu") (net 2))
 (segment (start 130.774215 7.995) (end 138.927 7.995) (width 0.2) (layer "B.Cu") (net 2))
 (segment (start 123.168714 6.028) (end 127.978787 6.028) (width 0.2) (layer "B.Cu") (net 2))
 (segment (start 121.017893 7.764607) (end 122.461607 6.320893) (width 0.2) (layer "B.Cu") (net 2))
 (arc (start 122.461607 6.320893) (mid 122.78603 6.10412) (end 123.168714 6.028) (width 0.2) (layer "B.Cu") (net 2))
 (arc (start 130.067108 7.702107) (mid 130.391531 7.91888) (end 130.774215 7.995) (width 0.2) (layer "B.Cu") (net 2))
 (arc (start 120.725 8.471714) (mid 120.80112 8.089031) (end 121.017893 7.764607) (width 0.2) (layer "B.Cu") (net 2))
 (arc (start 128.685894 6.320893) (mid 128.361471 6.10412) (end 127.978787 6.028) (width 0.2) (layer "B.Cu") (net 2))
 (segment (start 121.525 9.0075) (end 121.525 8.471714) (width 0.2) (layer "B.Cu") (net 3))
 (segment (start 128.374893 6.983893) (end 130.093107 8.702107) (width 0.2) (layer "B.Cu") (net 3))
 (segment (start 121.817893 7.764607) (end 122.598607 6.983893) (width 0.2) (layer "B.Cu") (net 3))
 (segment (start 123.305714 6.691) (end 127.667786 6.691) (width 0.2) (layer "B.Cu") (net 3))
 (segment (start 130.800214 8.995) (end 138.927 8.995) (width 0.2) (layer "B.Cu") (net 3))
 (arc (start 121.817893 7.764607) (mid 121.60112 8.08903) (end 121.525 8.471714) (width 0.2) (layer "B.Cu") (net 3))
 (arc (start 130.800214 8.995) (mid 130.417531 8.91888) (end 130.093107 8.702107) (width 0.2) (layer "B.Cu") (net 3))
 (arc (start 122.598607 6.983893) (mid 122.92303 6.76712) (end 123.305714 6.691) (width 0.2) (layer "B.Cu") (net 3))
 (arc (start 127.667786 6.691) (mid 128.050469 6.76712) (end 128.374893 6.983893) (width 0.2) (layer "B.Cu") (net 3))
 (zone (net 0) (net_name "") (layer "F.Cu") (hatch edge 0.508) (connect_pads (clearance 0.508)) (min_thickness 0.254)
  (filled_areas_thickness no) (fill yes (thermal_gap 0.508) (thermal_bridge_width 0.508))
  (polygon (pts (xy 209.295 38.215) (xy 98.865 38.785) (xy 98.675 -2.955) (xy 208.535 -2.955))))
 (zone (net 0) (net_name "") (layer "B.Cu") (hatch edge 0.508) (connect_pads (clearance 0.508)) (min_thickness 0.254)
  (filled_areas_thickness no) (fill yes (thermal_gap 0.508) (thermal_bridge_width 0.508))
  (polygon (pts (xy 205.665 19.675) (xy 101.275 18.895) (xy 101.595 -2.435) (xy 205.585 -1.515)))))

